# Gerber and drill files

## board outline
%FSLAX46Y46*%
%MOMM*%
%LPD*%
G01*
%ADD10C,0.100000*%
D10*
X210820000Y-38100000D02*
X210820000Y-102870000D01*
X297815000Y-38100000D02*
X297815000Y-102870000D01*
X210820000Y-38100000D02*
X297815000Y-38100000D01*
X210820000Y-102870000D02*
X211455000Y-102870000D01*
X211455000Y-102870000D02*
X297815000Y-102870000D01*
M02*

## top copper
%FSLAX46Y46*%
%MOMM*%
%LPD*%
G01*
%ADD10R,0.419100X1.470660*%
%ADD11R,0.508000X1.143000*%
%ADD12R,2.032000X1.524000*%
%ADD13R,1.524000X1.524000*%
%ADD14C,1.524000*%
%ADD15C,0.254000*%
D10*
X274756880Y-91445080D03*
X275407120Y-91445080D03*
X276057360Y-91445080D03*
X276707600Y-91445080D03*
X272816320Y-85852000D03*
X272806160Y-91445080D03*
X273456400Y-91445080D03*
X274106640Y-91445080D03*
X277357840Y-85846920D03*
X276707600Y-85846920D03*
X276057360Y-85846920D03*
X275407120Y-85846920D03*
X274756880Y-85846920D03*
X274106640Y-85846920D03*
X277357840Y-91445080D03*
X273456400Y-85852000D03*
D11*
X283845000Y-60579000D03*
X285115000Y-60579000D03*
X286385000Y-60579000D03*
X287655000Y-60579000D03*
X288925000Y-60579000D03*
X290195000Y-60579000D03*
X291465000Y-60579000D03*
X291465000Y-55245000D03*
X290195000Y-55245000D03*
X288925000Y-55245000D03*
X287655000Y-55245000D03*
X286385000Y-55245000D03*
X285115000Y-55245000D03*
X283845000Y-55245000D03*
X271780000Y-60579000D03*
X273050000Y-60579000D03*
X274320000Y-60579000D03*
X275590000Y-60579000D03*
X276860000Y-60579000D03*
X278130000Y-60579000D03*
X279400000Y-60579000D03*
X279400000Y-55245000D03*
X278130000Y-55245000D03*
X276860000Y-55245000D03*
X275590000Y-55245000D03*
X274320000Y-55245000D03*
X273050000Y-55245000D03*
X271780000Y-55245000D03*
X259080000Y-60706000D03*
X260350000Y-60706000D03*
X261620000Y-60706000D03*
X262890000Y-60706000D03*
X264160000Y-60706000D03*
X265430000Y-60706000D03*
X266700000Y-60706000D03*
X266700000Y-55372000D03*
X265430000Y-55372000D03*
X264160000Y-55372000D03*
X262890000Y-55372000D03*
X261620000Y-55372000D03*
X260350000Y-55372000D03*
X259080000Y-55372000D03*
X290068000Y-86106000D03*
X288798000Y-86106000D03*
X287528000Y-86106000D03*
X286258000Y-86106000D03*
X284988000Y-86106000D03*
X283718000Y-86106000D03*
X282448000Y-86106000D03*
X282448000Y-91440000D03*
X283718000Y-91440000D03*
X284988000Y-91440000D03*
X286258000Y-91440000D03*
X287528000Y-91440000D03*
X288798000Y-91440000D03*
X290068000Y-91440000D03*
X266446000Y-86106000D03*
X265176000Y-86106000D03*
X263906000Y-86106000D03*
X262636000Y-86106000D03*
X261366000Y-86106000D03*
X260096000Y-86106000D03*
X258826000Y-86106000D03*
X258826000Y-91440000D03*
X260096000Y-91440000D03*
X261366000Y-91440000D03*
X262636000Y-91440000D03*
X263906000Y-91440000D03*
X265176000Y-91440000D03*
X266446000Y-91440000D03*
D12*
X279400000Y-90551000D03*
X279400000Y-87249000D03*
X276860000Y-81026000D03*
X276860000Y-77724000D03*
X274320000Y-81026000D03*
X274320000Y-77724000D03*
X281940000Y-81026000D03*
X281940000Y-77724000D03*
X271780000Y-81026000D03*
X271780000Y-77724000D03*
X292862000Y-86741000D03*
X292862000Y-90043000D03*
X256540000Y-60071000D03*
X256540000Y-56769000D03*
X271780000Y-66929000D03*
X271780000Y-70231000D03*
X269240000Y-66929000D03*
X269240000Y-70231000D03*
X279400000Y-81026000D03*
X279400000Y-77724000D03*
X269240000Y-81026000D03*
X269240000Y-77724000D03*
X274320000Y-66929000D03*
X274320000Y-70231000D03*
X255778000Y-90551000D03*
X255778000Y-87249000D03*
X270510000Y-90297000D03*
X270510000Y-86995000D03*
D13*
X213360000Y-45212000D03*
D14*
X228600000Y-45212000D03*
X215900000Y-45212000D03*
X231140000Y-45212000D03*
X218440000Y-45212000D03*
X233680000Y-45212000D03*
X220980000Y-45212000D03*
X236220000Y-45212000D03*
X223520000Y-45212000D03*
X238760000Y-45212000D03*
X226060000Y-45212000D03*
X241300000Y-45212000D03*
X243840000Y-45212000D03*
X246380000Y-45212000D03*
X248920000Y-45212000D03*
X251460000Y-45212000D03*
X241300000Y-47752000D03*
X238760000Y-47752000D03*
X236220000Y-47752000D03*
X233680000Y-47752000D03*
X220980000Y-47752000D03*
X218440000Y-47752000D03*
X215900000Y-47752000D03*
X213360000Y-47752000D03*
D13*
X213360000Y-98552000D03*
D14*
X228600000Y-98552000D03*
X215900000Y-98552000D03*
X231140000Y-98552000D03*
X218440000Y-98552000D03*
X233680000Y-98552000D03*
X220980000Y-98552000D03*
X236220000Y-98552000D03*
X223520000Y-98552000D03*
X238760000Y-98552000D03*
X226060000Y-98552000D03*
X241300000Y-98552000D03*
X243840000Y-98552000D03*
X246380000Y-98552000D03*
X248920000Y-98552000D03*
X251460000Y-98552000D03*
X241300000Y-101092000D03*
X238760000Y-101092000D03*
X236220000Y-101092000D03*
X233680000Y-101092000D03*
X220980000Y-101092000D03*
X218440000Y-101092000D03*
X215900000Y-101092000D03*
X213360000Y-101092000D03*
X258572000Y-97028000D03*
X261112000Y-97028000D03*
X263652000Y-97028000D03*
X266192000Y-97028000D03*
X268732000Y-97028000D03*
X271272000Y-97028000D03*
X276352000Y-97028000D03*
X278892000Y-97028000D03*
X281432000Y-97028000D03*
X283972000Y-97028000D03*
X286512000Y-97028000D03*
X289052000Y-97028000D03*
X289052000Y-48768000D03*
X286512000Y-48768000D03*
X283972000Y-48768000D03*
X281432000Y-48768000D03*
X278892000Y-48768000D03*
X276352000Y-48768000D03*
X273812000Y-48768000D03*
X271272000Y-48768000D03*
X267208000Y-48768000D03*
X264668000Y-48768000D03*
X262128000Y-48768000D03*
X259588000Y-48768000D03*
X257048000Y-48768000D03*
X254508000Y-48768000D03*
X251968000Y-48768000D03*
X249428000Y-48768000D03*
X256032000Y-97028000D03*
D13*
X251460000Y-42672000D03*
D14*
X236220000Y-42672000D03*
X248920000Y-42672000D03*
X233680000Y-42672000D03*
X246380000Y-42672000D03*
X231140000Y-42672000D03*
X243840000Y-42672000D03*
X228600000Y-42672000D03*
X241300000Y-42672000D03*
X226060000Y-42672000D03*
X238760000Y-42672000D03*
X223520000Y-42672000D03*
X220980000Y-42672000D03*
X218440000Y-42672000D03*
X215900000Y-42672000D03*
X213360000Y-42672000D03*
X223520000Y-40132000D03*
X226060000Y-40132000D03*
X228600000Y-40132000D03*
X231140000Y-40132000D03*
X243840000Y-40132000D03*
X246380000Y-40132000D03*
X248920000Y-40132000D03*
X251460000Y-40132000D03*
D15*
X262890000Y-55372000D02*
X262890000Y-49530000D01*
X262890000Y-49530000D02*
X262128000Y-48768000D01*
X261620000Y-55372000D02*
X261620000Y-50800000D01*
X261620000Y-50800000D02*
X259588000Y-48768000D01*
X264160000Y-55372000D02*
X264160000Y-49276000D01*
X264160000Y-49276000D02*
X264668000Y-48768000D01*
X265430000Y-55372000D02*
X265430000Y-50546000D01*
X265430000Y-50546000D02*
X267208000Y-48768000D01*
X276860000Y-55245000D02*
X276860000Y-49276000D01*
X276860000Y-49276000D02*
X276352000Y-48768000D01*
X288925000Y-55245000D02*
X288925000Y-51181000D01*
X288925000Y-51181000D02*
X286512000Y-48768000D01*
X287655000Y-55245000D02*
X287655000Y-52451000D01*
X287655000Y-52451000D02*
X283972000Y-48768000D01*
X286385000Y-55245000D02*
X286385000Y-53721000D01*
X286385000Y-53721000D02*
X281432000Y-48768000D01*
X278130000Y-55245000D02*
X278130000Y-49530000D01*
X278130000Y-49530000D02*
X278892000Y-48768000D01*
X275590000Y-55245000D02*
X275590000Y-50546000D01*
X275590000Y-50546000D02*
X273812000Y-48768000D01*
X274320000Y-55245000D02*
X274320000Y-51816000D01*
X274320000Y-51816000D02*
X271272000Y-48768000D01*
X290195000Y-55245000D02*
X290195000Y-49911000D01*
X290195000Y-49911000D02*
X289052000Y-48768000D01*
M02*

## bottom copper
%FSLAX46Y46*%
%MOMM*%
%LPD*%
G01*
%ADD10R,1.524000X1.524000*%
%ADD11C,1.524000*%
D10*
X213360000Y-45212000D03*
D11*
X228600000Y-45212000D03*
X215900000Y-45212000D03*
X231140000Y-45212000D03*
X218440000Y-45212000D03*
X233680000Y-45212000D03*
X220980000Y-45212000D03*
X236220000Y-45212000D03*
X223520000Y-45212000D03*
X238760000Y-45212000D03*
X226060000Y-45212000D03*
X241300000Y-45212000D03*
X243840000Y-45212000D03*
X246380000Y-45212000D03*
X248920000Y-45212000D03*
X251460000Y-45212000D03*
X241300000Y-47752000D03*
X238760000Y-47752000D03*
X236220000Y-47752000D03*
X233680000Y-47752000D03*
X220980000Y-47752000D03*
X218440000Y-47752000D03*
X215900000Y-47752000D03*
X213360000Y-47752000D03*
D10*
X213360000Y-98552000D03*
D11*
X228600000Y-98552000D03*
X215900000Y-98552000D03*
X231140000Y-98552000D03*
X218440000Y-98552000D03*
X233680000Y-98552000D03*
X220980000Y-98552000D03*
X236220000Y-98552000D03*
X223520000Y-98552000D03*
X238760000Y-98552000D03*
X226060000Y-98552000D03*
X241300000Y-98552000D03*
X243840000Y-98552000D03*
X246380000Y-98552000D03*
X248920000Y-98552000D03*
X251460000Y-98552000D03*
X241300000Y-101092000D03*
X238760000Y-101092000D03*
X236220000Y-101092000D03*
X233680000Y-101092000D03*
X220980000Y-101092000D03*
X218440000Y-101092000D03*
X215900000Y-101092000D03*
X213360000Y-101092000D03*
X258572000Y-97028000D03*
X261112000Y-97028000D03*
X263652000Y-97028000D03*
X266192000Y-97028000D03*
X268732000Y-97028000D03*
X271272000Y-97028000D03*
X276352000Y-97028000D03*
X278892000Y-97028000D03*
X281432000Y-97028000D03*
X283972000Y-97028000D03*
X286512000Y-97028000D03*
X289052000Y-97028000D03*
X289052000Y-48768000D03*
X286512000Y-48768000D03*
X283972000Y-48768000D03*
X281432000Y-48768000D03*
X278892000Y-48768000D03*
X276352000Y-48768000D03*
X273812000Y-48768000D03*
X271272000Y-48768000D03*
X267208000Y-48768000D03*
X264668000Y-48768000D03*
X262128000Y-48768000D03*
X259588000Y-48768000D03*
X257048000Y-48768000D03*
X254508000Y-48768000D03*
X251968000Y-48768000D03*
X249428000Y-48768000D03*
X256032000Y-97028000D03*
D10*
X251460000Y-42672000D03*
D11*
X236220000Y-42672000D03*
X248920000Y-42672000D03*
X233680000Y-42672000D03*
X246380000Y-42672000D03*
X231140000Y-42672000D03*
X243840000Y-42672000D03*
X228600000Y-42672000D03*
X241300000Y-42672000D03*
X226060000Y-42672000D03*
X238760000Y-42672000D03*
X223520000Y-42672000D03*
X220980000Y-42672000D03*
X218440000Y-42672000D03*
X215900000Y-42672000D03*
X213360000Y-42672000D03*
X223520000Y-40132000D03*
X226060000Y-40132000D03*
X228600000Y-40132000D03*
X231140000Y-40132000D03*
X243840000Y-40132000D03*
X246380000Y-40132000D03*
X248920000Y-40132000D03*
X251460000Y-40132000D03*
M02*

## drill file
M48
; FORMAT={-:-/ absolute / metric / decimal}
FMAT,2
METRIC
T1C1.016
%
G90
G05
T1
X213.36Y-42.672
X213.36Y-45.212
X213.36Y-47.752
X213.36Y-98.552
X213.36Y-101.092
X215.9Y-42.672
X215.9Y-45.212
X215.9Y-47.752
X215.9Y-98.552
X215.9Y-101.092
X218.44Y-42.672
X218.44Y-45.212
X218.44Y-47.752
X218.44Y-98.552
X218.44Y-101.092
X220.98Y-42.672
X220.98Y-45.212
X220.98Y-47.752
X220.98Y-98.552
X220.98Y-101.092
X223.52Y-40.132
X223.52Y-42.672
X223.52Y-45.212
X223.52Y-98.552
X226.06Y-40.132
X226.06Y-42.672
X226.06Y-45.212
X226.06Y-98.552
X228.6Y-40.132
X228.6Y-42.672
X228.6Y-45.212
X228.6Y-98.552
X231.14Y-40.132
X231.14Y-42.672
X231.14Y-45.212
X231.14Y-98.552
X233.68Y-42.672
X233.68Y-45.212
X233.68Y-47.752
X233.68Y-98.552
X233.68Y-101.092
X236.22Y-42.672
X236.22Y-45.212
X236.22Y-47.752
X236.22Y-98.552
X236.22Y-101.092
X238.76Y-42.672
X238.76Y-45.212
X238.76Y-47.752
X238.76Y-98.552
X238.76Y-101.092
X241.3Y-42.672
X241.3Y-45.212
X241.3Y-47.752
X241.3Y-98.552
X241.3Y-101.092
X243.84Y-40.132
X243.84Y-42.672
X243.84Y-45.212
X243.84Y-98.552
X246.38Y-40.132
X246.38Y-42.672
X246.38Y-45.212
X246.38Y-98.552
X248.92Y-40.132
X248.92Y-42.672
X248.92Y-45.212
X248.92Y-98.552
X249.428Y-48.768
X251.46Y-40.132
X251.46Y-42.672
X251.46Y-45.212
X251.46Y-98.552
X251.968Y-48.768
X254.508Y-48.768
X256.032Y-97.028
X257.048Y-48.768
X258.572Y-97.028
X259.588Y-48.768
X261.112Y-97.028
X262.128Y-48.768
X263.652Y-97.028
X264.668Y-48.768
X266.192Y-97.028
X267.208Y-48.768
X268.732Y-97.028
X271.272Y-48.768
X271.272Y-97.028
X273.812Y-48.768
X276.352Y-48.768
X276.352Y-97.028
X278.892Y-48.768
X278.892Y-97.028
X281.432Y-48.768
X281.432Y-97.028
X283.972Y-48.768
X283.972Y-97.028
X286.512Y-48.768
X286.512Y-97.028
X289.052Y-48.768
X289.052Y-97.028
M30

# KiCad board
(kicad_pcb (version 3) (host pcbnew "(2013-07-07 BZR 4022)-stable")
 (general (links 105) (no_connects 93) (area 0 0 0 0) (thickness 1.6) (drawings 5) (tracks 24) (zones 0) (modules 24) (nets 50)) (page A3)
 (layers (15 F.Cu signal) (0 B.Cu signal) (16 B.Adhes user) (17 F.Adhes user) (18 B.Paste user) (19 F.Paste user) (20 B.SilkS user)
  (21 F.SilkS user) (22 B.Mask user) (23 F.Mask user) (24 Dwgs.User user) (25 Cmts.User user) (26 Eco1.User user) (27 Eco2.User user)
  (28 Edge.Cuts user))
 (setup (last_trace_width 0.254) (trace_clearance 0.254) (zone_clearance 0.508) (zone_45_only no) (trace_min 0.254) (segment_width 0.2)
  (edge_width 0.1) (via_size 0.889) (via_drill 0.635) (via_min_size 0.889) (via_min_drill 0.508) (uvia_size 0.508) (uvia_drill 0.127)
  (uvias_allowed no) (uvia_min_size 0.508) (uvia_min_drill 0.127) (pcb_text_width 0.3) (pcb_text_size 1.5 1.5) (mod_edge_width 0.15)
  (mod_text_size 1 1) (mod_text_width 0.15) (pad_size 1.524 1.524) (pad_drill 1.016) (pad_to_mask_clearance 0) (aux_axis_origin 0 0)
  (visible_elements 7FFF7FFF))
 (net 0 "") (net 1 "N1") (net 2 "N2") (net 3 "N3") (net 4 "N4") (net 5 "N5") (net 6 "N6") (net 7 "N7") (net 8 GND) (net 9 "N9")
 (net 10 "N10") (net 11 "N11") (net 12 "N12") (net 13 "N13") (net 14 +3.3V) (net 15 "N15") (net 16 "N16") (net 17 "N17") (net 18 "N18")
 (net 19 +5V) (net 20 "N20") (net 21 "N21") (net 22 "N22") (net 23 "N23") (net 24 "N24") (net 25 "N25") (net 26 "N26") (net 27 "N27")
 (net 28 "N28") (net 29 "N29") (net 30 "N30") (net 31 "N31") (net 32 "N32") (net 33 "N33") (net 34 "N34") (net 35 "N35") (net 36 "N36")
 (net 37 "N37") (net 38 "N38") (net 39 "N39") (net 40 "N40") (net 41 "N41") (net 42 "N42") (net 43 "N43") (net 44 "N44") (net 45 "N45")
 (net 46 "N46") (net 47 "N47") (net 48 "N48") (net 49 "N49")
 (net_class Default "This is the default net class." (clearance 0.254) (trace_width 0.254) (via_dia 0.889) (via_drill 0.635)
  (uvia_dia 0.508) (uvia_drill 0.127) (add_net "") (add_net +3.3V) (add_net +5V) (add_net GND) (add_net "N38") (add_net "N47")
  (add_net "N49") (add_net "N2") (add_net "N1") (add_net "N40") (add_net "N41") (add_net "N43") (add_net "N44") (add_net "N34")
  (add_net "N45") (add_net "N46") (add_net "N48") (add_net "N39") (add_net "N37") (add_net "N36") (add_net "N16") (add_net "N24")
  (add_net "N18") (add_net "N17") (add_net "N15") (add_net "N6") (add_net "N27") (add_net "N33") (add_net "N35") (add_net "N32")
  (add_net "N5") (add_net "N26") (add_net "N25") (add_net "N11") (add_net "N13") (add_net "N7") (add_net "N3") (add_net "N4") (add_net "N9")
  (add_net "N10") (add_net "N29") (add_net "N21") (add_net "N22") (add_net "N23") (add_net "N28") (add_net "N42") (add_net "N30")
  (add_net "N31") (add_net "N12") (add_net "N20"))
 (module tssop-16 (layer F.Cu) (at 275.082 88.646)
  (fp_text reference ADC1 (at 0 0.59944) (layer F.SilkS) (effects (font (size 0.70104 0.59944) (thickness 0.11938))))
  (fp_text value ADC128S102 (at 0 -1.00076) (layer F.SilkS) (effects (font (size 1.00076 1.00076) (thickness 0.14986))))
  (pad 4 smd rect (at -0.32512 2.79908) (size 0.4191 1.47066) (layers F.Cu F.Paste F.Mask) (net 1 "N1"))
  (pad 5 smd rect (at 0.32512 2.79908) (size 0.4191 1.47066) (layers F.Cu F.Paste F.Mask) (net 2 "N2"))
  (pad 6 smd rect (at 0.97536 2.79908) (size 0.4191 1.47066) (layers F.Cu F.Paste F.Mask) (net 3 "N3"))
  (pad 7 smd rect (at 1.6256 2.79908) (size 0.4191 1.47066) (layers F.Cu F.Paste F.Mask) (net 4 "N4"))
  (pad 16 smd rect (at -2.26568 -2.794) (size 0.4191 1.47066) (layers F.Cu F.Paste F.Mask) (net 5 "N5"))
  (pad 1 smd rect (at -2.27584 2.79908) (size 0.4191 1.47066) (layers F.Cu F.Paste F.Mask) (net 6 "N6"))
  (pad 2 smd rect (at -1.6256 2.79908) (size 0.4191 1.47066) (layers F.Cu F.Paste F.Mask) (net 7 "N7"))
  (pad 3 smd rect (at -0.97536 2.79908) (size 0.4191 1.47066) (layers F.Cu F.Paste F.Mask) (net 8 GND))
  (pad 9 smd rect (at 2.27584 -2.79908) (size 0.4191 1.47066) (layers F.Cu F.Paste F.Mask) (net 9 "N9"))
  (pad 10 smd rect (at 1.6256 -2.79908) (size 0.4191 1.47066) (layers F.Cu F.Paste F.Mask))
  (pad 11 smd rect (at 0.97536 -2.79908) (size 0.4191 1.47066) (layers F.Cu F.Paste F.Mask))
  (pad 12 smd rect (at 0.32512 -2.79908) (size 0.4191 1.47066) (layers F.Cu F.Paste F.Mask) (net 8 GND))
  (pad 13 smd rect (at -0.32512 -2.79908) (size 0.4191 1.47066) (layers F.Cu F.Paste F.Mask) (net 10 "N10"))
  (pad 14 smd rect (at -0.97536 -2.79908) (size 0.4191 1.47066) (layers F.Cu F.Paste F.Mask) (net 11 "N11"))
  (pad 8 smd rect (at 2.27584 2.79908) (size 0.4191 1.47066) (layers F.Cu F.Paste F.Mask) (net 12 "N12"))
  (pad 15 smd rect (at -1.6256 -2.794) (size 0.4191 1.47066) (layers F.Cu F.Paste F.Mask) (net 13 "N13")))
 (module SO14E (layer F.Cu) (at 287.655 57.785)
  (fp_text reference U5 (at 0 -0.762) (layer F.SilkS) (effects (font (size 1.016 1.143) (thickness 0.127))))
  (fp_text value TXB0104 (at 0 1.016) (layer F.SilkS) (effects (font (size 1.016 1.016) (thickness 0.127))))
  (pad 1 smd rect (at -3.81 2.794) (size 0.508 1.143) (layers F.Cu F.Paste F.Mask) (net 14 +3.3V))
  (pad 2 smd rect (at -2.54 2.794) (size 0.508 1.143) (layers F.Cu F.Paste F.Mask) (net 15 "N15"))
  (pad 3 smd rect (at -1.27 2.794) (size 0.508 1.143) (layers F.Cu F.Paste F.Mask) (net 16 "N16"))
  (pad 4 smd rect (at 0 2.794) (size 0.508 1.143) (layers F.Cu F.Paste F.Mask) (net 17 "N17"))
  (pad 5 smd rect (at 1.27 2.794) (size 0.508 1.143) (layers F.Cu F.Paste F.Mask) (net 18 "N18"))
  (pad 6 smd rect (at 2.54 2.794) (size 0.508 1.143) (layers F.Cu F.Paste F.Mask))
  (pad 7 smd rect (at 3.81 2.794) (size 0.508 1.143) (layers F.Cu F.Paste F.Mask) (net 8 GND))
  (pad 8 smd rect (at 3.81 -2.54) (size 0.508 1.143) (layers F.Cu F.Paste F.Mask) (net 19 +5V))
  (pad 9 smd rect (at 2.54 -2.54) (size 0.508 1.143) (layers F.Cu F.Paste F.Mask) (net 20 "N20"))
  (pad 10 smd rect (at 1.27 -2.54) (size 0.508 1.143) (layers F.Cu F.Paste F.Mask) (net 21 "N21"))
  (pad 11 smd rect (at 0 -2.54) (size 0.508 1.143) (layers F.Cu F.Paste F.Mask) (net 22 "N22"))
  (pad 12 smd rect (at -1.27 -2.54) (size 0.508 1.143) (layers F.Cu F.Paste F.Mask) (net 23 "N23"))
  (pad 13 smd rect (at -2.54 -2.54) (size 0.508 1.143) (layers F.Cu F.Paste F.Mask))
  (pad 14 smd rect (at -3.81 -2.54) (size 0.508 1.143) (layers F.Cu F.Paste F.Mask)))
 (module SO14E (layer F.Cu) (at 275.59 57.785)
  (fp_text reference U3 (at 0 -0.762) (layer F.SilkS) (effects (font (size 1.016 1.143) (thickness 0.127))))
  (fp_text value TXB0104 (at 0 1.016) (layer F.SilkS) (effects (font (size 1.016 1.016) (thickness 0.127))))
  (pad 1 smd rect (at -3.81 2.794) (size 0.508 1.143) (layers F.Cu F.Paste F.Mask) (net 14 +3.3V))
  (pad 2 smd rect (at -2.54 2.794) (size 0.508 1.143) (layers F.Cu F.Paste F.Mask) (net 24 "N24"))
  (pad 3 smd rect (at -1.27 2.794) (size 0.508 1.143) (layers F.Cu F.Paste F.Mask) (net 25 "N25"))
  (pad 4 smd rect (at 0 2.794) (size 0.508 1.143) (layers F.Cu F.Paste F.Mask) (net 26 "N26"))
  (pad 5 smd rect (at 1.27 2.794) (size 0.508 1.143) (layers F.Cu F.Paste F.Mask) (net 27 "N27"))
  (pad 6 smd rect (at 2.54 2.794) (size 0.508 1.143) (layers F.Cu F.Paste F.Mask))
  (pad 7 smd rect (at 3.81 2.794) (size 0.508 1.143) (layers F.Cu F.Paste F.Mask) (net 8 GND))
  (pad 8 smd rect (at 3.81 -2.54) (size 0.508 1.143) (layers F.Cu F.Paste F.Mask) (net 19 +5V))
  (pad 9 smd rect (at 2.54 -2.54) (size 0.508 1.143) (layers F.Cu F.Paste F.Mask) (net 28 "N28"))
  (pad 10 smd rect (at 1.27 -2.54) (size 0.508 1.143) (layers F.Cu F.Paste F.Mask) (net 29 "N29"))
  (pad 11 smd rect (at 0 -2.54) (size 0.508 1.143) (layers F.Cu F.Paste F.Mask) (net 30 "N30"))
  (pad 12 smd rect (at -1.27 -2.54) (size 0.508 1.143) (layers F.Cu F.Paste F.Mask) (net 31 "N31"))
  (pad 13 smd rect (at -2.54 -2.54) (size 0.508 1.143) (layers F.Cu F.Paste F.Mask))
  (pad 14 smd rect (at -3.81 -2.54) (size 0.508 1.143) (layers F.Cu F.Paste F.Mask)))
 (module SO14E (layer F.Cu) (at 262.89 57.912)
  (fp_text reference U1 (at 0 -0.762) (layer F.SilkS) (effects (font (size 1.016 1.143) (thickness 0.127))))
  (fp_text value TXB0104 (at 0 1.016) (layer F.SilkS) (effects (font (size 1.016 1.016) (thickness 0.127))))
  (pad 1 smd rect (at -3.81 2.794) (size 0.508 1.143) (layers F.Cu F.Paste F.Mask) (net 14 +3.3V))
  (pad 2 smd rect (at -2.54 2.794) (size 0.508 1.143) (layers F.Cu F.Paste F.Mask) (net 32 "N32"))
  (pad 3 smd rect (at -1.27 2.794) (size 0.508 1.143) (layers F.Cu F.Paste F.Mask) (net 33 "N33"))
  (pad 4 smd rect (at 0 2.794) (size 0.508 1.143) (layers F.Cu F.Paste F.Mask) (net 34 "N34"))
  (pad 5 smd rect (at 1.27 2.794) (size 0.508 1.143) (layers F.Cu F.Paste F.Mask) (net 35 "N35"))
  (pad 6 smd rect (at 2.54 2.794) (size 0.508 1.143) (layers F.Cu F.Paste F.Mask))
  (pad 7 smd rect (at 3.81 2.794) (size 0.508 1.143) (layers F.Cu F.Paste F.Mask))
  (pad 8 smd rect (at 3.81 -2.54) (size 0.508 1.143) (layers F.Cu F.Paste F.Mask) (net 19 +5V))
  (pad 9 smd rect (at 2.54 -2.54) (size 0.508 1.143) (layers F.Cu F.Paste F.Mask) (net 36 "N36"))
  (pad 10 smd rect (at 1.27 -2.54) (size 0.508 1.143) (layers F.Cu F.Paste F.Mask) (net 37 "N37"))
  (pad 11 smd rect (at 0 -2.54) (size 0.508 1.143) (layers F.Cu F.Paste F.Mask) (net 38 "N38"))
  (pad 12 smd rect (at -1.27 -2.54) (size 0.508 1.143) (layers F.Cu F.Paste F.Mask) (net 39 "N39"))
  (pad 13 smd rect (at -2.54 -2.54) (size 0.508 1.143) (layers F.Cu F.Paste F.Mask))
  (pad 14 smd rect (at -3.81 -2.54) (size 0.508 1.143) (layers F.Cu F.Paste F.Mask)))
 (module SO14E (layer F.Cu) (at 286.258 88.9 180)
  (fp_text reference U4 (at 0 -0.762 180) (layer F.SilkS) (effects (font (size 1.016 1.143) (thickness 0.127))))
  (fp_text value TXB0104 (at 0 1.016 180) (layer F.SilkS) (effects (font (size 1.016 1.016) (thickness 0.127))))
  (pad 1 smd rect (at -3.81 2.794 180) (size 0.508 1.143) (layers F.Cu F.Paste F.Mask) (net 14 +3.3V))
  (pad 2 smd rect (at -2.54 2.794 180) (size 0.508 1.143) (layers F.Cu F.Paste F.Mask) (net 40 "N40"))
  (pad 3 smd rect (at -1.27 2.794 180) (size 0.508 1.143) (layers F.Cu F.Paste F.Mask) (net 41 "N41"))
  (pad 4 smd rect (at 0 2.794 180) (size 0.508 1.143) (layers F.Cu F.Paste F.Mask) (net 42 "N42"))
  (pad 5 smd rect (at 1.27 2.794 180) (size 0.508 1.143) (layers F.Cu F.Paste F.Mask) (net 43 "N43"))
  (pad 6 smd rect (at 2.54 2.794 180) (size 0.508 1.143) (layers F.Cu F.Paste F.Mask))
  (pad 7 smd rect (at 3.81 2.794 180) (size 0.508 1.143) (layers F.Cu F.Paste F.Mask) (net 8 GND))
  (pad 8 smd rect (at 3.81 -2.54 180) (size 0.508 1.143) (layers F.Cu F.Paste F.Mask) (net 19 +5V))
  (pad 9 smd rect (at 2.54 -2.54 180) (size 0.508 1.143) (layers F.Cu F.Paste F.Mask) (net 3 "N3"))
  (pad 10 smd rect (at 1.27 -2.54 180) (size 0.508 1.143) (layers F.Cu F.Paste F.Mask) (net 4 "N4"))
  (pad 11 smd rect (at 0 -2.54 180) (size 0.508 1.143) (layers F.Cu F.Paste F.Mask) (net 12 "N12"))
  (pad 12 smd rect (at -1.27 -2.54 180) (size 0.508 1.143) (layers F.Cu F.Paste F.Mask) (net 9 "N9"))
  (pad 13 smd rect (at -2.54 -2.54 180) (size 0.508 1.143) (layers F.Cu F.Paste F.Mask))
  (pad 14 smd rect (at -3.81 -2.54 180) (size 0.508 1.143) (layers F.Cu F.Paste F.Mask)))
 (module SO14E (layer F.Cu) (at 262.636 88.9 180)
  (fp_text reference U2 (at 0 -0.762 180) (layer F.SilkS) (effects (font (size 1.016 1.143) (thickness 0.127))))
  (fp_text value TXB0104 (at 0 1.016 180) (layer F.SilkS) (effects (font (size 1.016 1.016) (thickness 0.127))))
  (pad 1 smd rect (at -3.81 2.794 180) (size 0.508 1.143) (layers F.Cu F.Paste F.Mask) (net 14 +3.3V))
  (pad 2 smd rect (at -2.54 2.794 180) (size 0.508 1.143) (layers F.Cu F.Paste F.Mask) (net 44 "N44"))
  (pad 3 smd rect (at -1.27 2.794 180) (size 0.508 1.143) (layers F.Cu F.Paste F.Mask) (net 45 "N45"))
  (pad 4 smd rect (at 0 2.794 180) (size 0.508 1.143) (layers F.Cu F.Paste F.Mask) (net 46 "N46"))
  (pad 5 smd rect (at 1.27 2.794 180) (size 0.508 1.143) (layers F.Cu F.Paste F.Mask) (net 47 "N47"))
  (pad 6 smd rect (at 2.54 2.794 180) (size 0.508 1.143) (layers F.Cu F.Paste F.Mask))
  (pad 7 smd rect (at 3.81 2.794 180) (size 0.508 1.143) (layers F.Cu F.Paste F.Mask) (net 8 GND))
  (pad 8 smd rect (at 3.81 -2.54 180) (size 0.508 1.143) (layers F.Cu F.Paste F.Mask) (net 19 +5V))
  (pad 9 smd rect (at 2.54 -2.54 180) (size 0.508 1.143) (layers F.Cu F.Paste F.Mask) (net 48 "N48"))
  (pad 10 smd rect (at 1.27 -2.54 180) (size 0.508 1.143) (layers F.Cu F.Paste F.Mask) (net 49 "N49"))
  (pad 11 smd rect (at 0 -2.54 180) (size 0.508 1.143) (layers F.Cu F.Paste F.Mask) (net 1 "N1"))
  (pad 12 smd rect (at -1.27 -2.54 180) (size 0.508 1.143) (layers F.Cu F.Paste F.Mask) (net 2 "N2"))
  (pad 13 smd rect (at -2.54 -2.54 180) (size 0.508 1.143) (layers F.Cu F.Paste F.Mask))
  (pad 14 smd rect (at -3.81 -2.54 180) (size 0.508 1.143) (layers F.Cu F.Paste F.Mask)))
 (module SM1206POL (layer F.Cu) (at 279.4 88.9 90)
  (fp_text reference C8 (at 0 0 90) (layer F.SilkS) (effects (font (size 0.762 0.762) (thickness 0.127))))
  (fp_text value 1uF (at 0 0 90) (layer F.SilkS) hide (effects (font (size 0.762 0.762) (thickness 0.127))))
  (pad 1 smd rect (at -1.651 0 90) (size 1.524 2.032) (layers F.Cu F.Paste F.Mask) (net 7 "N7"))
  (pad 2 smd rect (at 1.651 0 90) (size 1.524 2.032) (layers F.Cu F.Paste F.Mask) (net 8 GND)))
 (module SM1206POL (layer F.Cu) (at 276.86 79.375 90)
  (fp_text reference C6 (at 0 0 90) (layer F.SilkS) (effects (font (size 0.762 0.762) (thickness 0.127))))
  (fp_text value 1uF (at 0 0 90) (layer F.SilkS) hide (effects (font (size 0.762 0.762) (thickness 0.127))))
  (pad 1 smd rect (at -1.651 0 90) (size 1.524 2.032) (layers F.Cu F.Paste F.Mask) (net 10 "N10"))
  (pad 2 smd rect (at 1.651 0 90) (size 1.524 2.032) (layers F.Cu F.Paste F.Mask) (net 8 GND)))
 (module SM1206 (layer F.Cu) (at 274.32 79.375 90)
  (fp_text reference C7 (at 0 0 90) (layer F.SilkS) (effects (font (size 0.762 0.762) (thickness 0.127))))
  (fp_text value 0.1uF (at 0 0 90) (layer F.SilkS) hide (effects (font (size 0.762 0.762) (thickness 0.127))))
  (pad 1 smd rect (at -1.651 0 90) (size 1.524 2.032) (layers F.Cu F.Paste F.Mask) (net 10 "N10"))
  (pad 2 smd rect (at 1.651 0 90) (size 1.524 2.032) (layers F.Cu F.Paste F.Mask) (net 8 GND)))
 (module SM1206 (layer F.Cu) (at 281.94 79.375 90)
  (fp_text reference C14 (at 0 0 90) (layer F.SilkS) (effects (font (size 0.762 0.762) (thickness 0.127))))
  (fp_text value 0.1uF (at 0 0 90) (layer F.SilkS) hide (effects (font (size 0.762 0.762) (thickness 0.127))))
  (pad 1 smd rect (at -1.651 0 90) (size 1.524 2.032) (layers F.Cu F.Paste F.Mask) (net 14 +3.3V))
  (pad 2 smd rect (at 1.651 0 90) (size 1.524 2.032) (layers F.Cu F.Paste F.Mask) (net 8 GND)))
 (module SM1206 (layer F.Cu) (at 271.78 79.375 90)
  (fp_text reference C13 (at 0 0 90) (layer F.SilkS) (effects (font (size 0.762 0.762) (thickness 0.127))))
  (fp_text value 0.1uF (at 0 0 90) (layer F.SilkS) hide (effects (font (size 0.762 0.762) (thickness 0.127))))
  (pad 1 smd rect (at -1.651 0 90) (size 1.524 2.032) (layers F.Cu F.Paste F.Mask) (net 14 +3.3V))
  (pad 2 smd rect (at 1.651 0 90) (size 1.524 2.032) (layers F.Cu F.Paste F.Mask) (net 8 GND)))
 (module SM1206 (layer F.Cu) (at 292.862 88.392 270)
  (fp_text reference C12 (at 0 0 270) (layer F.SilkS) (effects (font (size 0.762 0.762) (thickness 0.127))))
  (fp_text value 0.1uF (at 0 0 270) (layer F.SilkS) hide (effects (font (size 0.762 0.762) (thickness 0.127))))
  (pad 1 smd rect (at -1.651 0 270) (size 1.524 2.032) (layers F.Cu F.Paste F.Mask) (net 14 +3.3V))
  (pad 2 smd rect (at 1.651 0 270) (size 1.524 2.032) (layers F.Cu F.Paste F.Mask) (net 8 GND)))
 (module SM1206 (layer F.Cu) (at 256.54 58.42 90)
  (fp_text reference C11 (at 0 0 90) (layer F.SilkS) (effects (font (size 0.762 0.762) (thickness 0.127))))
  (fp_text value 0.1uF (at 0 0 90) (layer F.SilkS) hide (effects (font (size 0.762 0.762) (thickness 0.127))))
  (pad 1 smd rect (at -1.651 0 90) (size 1.524 2.032) (layers F.Cu F.Paste F.Mask) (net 14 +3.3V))
  (pad 2 smd rect (at 1.651 0 90) (size 1.524 2.032) (layers F.Cu F.Paste F.Mask) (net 8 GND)))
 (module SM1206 (layer F.Cu) (at 271.78 68.58 270)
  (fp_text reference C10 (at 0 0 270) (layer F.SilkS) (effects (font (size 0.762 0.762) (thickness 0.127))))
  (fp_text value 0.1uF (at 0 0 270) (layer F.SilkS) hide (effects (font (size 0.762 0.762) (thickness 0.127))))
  (pad 1 smd rect (at -1.651 0 270) (size 1.524 2.032) (layers F.Cu F.Paste F.Mask) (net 14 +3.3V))
  (pad 2 smd rect (at 1.651 0 270) (size 1.524 2.032) (layers F.Cu F.Paste F.Mask) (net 8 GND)))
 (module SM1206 (layer F.Cu) (at 269.24 68.58 270)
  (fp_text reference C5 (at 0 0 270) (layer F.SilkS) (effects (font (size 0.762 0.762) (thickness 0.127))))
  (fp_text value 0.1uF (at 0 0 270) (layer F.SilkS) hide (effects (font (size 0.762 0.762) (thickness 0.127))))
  (pad 1 smd rect (at -1.651 0 270) (size 1.524 2.032) (layers F.Cu F.Paste F.Mask) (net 19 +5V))
  (pad 2 smd rect (at 1.651 0 270) (size 1.524 2.032) (layers F.Cu F.Paste F.Mask) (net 8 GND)))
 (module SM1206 (layer F.Cu) (at 279.4 79.375 90)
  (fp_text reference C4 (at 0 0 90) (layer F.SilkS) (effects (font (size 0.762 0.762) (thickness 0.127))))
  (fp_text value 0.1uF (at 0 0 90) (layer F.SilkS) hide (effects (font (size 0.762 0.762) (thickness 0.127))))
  (pad 1 smd rect (at -1.651 0 90) (size 1.524 2.032) (layers F.Cu F.Paste F.Mask) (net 19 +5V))
  (pad 2 smd rect (at 1.651 0 90) (size 1.524 2.032) (layers F.Cu F.Paste F.Mask) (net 8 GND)))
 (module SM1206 (layer F.Cu) (at 269.24 79.375 90)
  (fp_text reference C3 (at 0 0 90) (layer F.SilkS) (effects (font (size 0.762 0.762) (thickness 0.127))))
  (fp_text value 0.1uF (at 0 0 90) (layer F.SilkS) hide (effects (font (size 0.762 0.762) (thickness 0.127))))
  (pad 1 smd rect (at -1.651 0 90) (size 1.524 2.032) (layers F.Cu F.Paste F.Mask) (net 19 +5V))
  (pad 2 smd rect (at 1.651 0 90) (size 1.524 2.032) (layers F.Cu F.Paste F.Mask) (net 8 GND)))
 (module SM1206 (layer F.Cu) (at 274.32 68.58 270)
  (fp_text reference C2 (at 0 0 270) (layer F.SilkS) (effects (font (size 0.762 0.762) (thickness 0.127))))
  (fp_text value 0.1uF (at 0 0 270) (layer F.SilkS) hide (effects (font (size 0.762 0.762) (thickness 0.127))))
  (pad 1 smd rect (at -1.651 0 270) (size 1.524 2.032) (layers F.Cu F.Paste F.Mask) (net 19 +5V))
  (pad 2 smd rect (at 1.651 0 270) (size 1.524 2.032) (layers F.Cu F.Paste F.Mask) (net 8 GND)))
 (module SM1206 (layer F.Cu) (at 255.778 88.9 90)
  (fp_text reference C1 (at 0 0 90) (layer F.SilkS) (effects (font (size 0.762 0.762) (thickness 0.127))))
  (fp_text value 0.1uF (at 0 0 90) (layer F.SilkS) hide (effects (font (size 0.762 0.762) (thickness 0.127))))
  (pad 1 smd rect (at -1.651 0 90) (size 1.524 2.032) (layers F.Cu F.Paste F.Mask) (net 19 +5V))
  (pad 2 smd rect (at 1.651 0 90) (size 1.524 2.032) (layers F.Cu F.Paste F.Mask) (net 8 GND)))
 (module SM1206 (layer F.Cu) (at 270.51 88.646 90)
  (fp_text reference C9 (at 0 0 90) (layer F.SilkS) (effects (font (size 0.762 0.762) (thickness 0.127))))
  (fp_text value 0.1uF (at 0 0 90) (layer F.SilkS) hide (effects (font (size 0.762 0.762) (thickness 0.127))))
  (pad 1 smd rect (at -1.651 0 90) (size 1.524 2.032) (layers F.Cu F.Paste F.Mask) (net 7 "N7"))
  (pad 2 smd rect (at 1.651 0 90) (size 1.524 2.032) (layers F.Cu F.Paste F.Mask) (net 8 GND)))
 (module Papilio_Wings (layer F.Cu) (at 234.95 46.482)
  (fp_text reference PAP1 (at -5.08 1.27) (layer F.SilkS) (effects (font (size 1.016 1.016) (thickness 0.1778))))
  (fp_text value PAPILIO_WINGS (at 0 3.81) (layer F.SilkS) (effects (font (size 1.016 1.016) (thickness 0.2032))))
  (pad 1 thru_hole rect (at -21.59 -1.27) (size 1.524 1.524) (drill 1.016) (layers *.Cu *.Mask F.SilkS) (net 35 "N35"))
  (pad 7 thru_hole circle (at -6.35 -1.27) (size 1.524 1.524) (drill 1.016) (layers *.Cu *.Mask F.SilkS) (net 25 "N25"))
  (pad 2 thru_hole circle (at -19.05 -1.27) (size 1.524 1.524) (drill 1.016) (layers *.Cu *.Mask F.SilkS) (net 34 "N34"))
  (pad 8 thru_hole circle (at -3.81 -1.27) (size 1.524 1.524) (drill 1.016) (layers *.Cu *.Mask F.SilkS) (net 24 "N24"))
  (pad 3 thru_hole circle (at -16.51 -1.27) (size 1.524 1.524) (drill 1.016) (layers *.Cu *.Mask F.SilkS) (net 33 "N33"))
  (pad 9 thru_hole circle (at -1.27 -1.27) (size 1.524 1.524) (drill 1.016) (layers *.Cu *.Mask F.SilkS) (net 18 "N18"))
  (pad 4 thru_hole circle (at -13.97 -1.27) (size 1.524 1.524) (drill 1.016) (layers *.Cu *.Mask F.SilkS) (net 32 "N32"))
  (pad 10 thru_hole circle (at 1.27 -1.27) (size 1.524 1.524) (drill 1.016) (layers *.Cu *.Mask F.SilkS) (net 17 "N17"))
  (pad 5 thru_hole circle (at -11.43 -1.27) (size 1.524 1.524) (drill 1.016) (layers *.Cu *.Mask F.SilkS) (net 27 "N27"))
  (pad 11 thru_hole circle (at 3.81 -1.27) (size 1.524 1.524) (drill 1.016) (layers *.Cu *.Mask F.SilkS) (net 16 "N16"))
  (pad 6 thru_hole circle (at -8.89 -1.27) (size 1.524 1.524) (drill 1.016) (layers *.Cu *.Mask F.SilkS) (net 26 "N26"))
  (pad 12 thru_hole circle (at 6.35 -1.27) (size 1.524 1.524) (drill 1.016) (layers *.Cu *.Mask F.SilkS) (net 15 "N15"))
  (pad 13 thru_hole circle (at 8.89 -1.27) (size 1.524 1.524) (drill 1.016) (layers *.Cu *.Mask F.SilkS))
  (pad 14 thru_hole circle (at 11.43 -1.27) (size 1.524 1.524) (drill 1.016) (layers *.Cu *.Mask F.SilkS))
  (pad 15 thru_hole circle (at 13.97 -1.27) (size 1.524 1.524) (drill 1.016) (layers *.Cu *.Mask F.SilkS))
  (pad 16 thru_hole circle (at 16.51 -1.27) (size 1.524 1.524) (drill 1.016) (layers *.Cu *.Mask F.SilkS))
  (pad 17 thru_hole circle (at 6.35 1.27) (size 1.524 1.524) (drill 1.016) (layers *.Cu *.Mask F.SilkS) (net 19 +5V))
  (pad 18 thru_hole circle (at 3.81 1.27) (size 1.524 1.524) (drill 1.016) (layers *.Cu *.Mask F.SilkS) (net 14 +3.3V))
  (pad 19 thru_hole circle (at 1.27 1.27) (size 1.524 1.524) (drill 1.016) (layers *.Cu *.Mask F.SilkS))
  (pad 20 thru_hole circle (at -1.27 1.27) (size 1.524 1.524) (drill 1.016) (layers *.Cu *.Mask F.SilkS) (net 8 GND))
  (pad 21 thru_hole circle (at -13.97 1.27) (size 1.524 1.524) (drill 1.016) (layers *.Cu *.Mask F.SilkS) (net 19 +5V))
  (pad 22 thru_hole circle (at -16.51 1.27) (size 1.524 1.524) (drill 1.016) (layers *.Cu *.Mask F.SilkS))
  (pad 23 thru_hole circle (at -19.05 1.27) (size 1.524 1.524) (drill 1.016) (layers *.Cu *.Mask F.SilkS) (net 14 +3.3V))
  (pad 24 thru_hole circle (at -21.59 1.27) (size 1.524 1.524) (drill 1.016) (layers *.Cu *.Mask F.SilkS) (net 8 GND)))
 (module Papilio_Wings (layer F.Cu) (at 234.95 99.822)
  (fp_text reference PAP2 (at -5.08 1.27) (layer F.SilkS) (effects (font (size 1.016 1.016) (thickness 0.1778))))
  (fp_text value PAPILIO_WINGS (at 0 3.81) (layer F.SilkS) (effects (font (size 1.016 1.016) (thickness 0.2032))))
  (pad 1 thru_hole rect (at -21.59 -1.27) (size 1.524 1.524) (drill 1.016) (layers *.Cu *.Mask F.SilkS))
  (pad 7 thru_hole circle (at -6.35 -1.27) (size 1.524 1.524) (drill 1.016) (layers *.Cu *.Mask F.SilkS) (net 5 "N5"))
  (pad 2 thru_hole circle (at -19.05 -1.27) (size 1.524 1.524) (drill 1.016) (layers *.Cu *.Mask F.SilkS))
  (pad 8 thru_hole circle (at -3.81 -1.27) (size 1.524 1.524) (drill 1.016) (layers *.Cu *.Mask F.SilkS) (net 6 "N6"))
  (pad 3 thru_hole circle (at -16.51 -1.27) (size 1.524 1.524) (drill 1.016) (layers *.Cu *.Mask F.SilkS))
  (pad 9 thru_hole circle (at -1.27 -1.27) (size 1.524 1.524) (drill 1.016) (layers *.Cu *.Mask F.SilkS) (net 43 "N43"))
  (pad 4 thru_hole circle (at -13.97 -1.27) (size 1.524 1.524) (drill 1.016) (layers *.Cu *.Mask F.SilkS))
  (pad 10 thru_hole circle (at 1.27 -1.27) (size 1.524 1.524) (drill 1.016) (layers *.Cu *.Mask F.SilkS) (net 42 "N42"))
  (pad 5 thru_hole circle (at -11.43 -1.27) (size 1.524 1.524) (drill 1.016) (layers *.Cu *.Mask F.SilkS) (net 13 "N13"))
  (pad 11 thru_hole circle (at 3.81 -1.27) (size 1.524 1.524) (drill 1.016) (layers *.Cu *.Mask F.SilkS) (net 41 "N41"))
  (pad 6 thru_hole circle (at -8.89 -1.27) (size 1.524 1.524) (drill 1.016) (layers *.Cu *.Mask F.SilkS) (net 11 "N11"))
  (pad 12 thru_hole circle (at 6.35 -1.27) (size 1.524 1.524) (drill 1.016) (layers *.Cu *.Mask F.SilkS) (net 40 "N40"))
  (pad 13 thru_hole circle (at 8.89 -1.27) (size 1.524 1.524) (drill 1.016) (layers *.Cu *.Mask F.SilkS) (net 47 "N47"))
  (pad 14 thru_hole circle (at 11.43 -1.27) (size 1.524 1.524) (drill 1.016) (layers *.Cu *.Mask F.SilkS) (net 46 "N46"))
  (pad 15 thru_hole circle (at 13.97 -1.27) (size 1.524 1.524) (drill 1.016) (layers *.Cu *.Mask F.SilkS) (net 45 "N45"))
  (pad 16 thru_hole circle (at 16.51 -1.27) (size 1.524 1.524) (drill 1.016) (layers *.Cu *.Mask F.SilkS) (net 44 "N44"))
  (pad 17 thru_hole circle (at 6.35 1.27) (size 1.524 1.524) (drill 1.016) (layers *.Cu *.Mask F.SilkS) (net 19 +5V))
  (pad 18 thru_hole circle (at 3.81 1.27) (size 1.524 1.524) (drill 1.016) (layers *.Cu *.Mask F.SilkS) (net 14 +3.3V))
  (pad 19 thru_hole circle (at 1.27 1.27) (size 1.524 1.524) (drill 1.016) (layers *.Cu *.Mask F.SilkS))
  (pad 20 thru_hole circle (at -1.27 1.27) (size 1.524 1.524) (drill 1.016) (layers *.Cu *.Mask F.SilkS) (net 8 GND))
  (pad 21 thru_hole circle (at -13.97 1.27) (size 1.524 1.524) (drill 1.016) (layers *.Cu *.Mask F.SilkS) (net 19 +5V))
  (pad 22 thru_hole circle (at -16.51 1.27) (size 1.524 1.524) (drill 1.016) (layers *.Cu *.Mask F.SilkS) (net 14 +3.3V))
  (pad 23 thru_hole circle (at -19.05 1.27) (size 1.524 1.524) (drill 1.016) (layers *.Cu *.Mask F.SilkS))
  (pad 24 thru_hole circle (at -21.59 1.27) (size 1.524 1.524) (drill 1.016) (layers *.Cu *.Mask F.SilkS) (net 8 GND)))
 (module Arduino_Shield (layer F.Cu) (at 271.272 72.644)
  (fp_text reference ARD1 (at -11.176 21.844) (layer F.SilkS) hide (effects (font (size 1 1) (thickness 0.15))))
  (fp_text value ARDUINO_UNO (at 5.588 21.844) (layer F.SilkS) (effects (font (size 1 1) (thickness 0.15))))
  (pad 2 thru_hole circle (at -12.7 24.384) (size 1.524 1.524) (drill 1.016) (layers *.Cu *.Mask F.SilkS))
  (pad 3 thru_hole circle (at -10.16 24.384) (size 1.524 1.524) (drill 1.016) (layers *.Cu *.Mask F.SilkS) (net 14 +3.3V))
  (pad 4 thru_hole circle (at -7.62 24.384) (size 1.524 1.524) (drill 1.016) (layers *.Cu *.Mask F.SilkS) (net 19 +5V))
  (pad 5 thru_hole circle (at -5.08 24.384) (size 1.524 1.524) (drill 1.016) (layers *.Cu *.Mask F.SilkS))
  (pad 6 thru_hole circle (at -2.54 24.384) (size 1.524 1.524) (drill 1.016) (layers *.Cu *.Mask F.SilkS))
  (pad 7 thru_hole circle (at 0 24.384) (size 1.524 1.524) (drill 1.016) (layers *.Cu *.Mask F.SilkS))
  (pad 8 thru_hole circle (at 5.08 24.384) (size 1.524 1.524) (drill 1.016) (layers *.Cu *.Mask F.SilkS) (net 1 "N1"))
  (pad 9 thru_hole circle (at 7.62 24.384) (size 1.524 1.524) (drill 1.016) (layers *.Cu *.Mask F.SilkS) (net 2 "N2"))
  (pad 10 thru_hole circle (at 10.16 24.384) (size 1.524 1.524) (drill 1.016) (layers *.Cu *.Mask F.SilkS) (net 3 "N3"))
  (pad 11 thru_hole circle (at 12.7 24.384) (size 1.524 1.524) (drill 1.016) (layers *.Cu *.Mask F.SilkS) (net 4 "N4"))
  (pad 12 thru_hole circle (at 15.24 24.384) (size 1.524 1.524) (drill 1.016) (layers *.Cu *.Mask F.SilkS) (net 12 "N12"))
  (pad 13 thru_hole circle (at 17.78 24.384) (size 1.524 1.524) (drill 1.016) (layers *.Cu *.Mask F.SilkS) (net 9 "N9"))
  (pad 14 thru_hole circle (at 17.78 -23.876) (size 1.524 1.524) (drill 1.016) (layers *.Cu *.Mask F.SilkS) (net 20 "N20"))
  (pad 15 thru_hole circle (at 15.24 -23.876) (size 1.524 1.524) (drill 1.016) (layers *.Cu *.Mask F.SilkS) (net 21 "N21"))
  (pad 16 thru_hole circle (at 12.7 -23.876) (size 1.524 1.524) (drill 1.016) (layers *.Cu *.Mask F.SilkS) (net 22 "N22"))
  (pad 17 thru_hole circle (at 10.16 -23.876) (size 1.524 1.524) (drill 1.016) (layers *.Cu *.Mask F.SilkS) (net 23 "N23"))
  (pad 18 thru_hole circle (at 7.62 -23.876) (size 1.524 1.524) (drill 1.016) (layers *.Cu *.Mask F.SilkS) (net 28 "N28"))
  (pad 19 thru_hole circle (at 5.08 -23.876) (size 1.524 1.524) (drill 1.016) (layers *.Cu *.Mask F.SilkS) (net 29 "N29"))
  (pad 20 thru_hole circle (at 2.54 -23.876) (size 1.524 1.524) (drill 1.016) (layers *.Cu *.Mask F.SilkS) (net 30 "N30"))
  (pad 21 thru_hole circle (at 0 -23.876) (size 1.524 1.524) (drill 1.016) (layers *.Cu *.Mask F.SilkS) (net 31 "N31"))
  (pad 22 thru_hole circle (at -4.064 -23.876) (size 1.524 1.524) (drill 1.016) (layers *.Cu *.Mask F.SilkS) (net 36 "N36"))
  (pad 23 thru_hole circle (at -6.604 -23.876) (size 1.524 1.524) (drill 1.016) (layers *.Cu *.Mask F.SilkS) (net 37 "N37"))
  (pad 24 thru_hole circle (at -9.144 -23.876) (size 1.524 1.524) (drill 1.016) (layers *.Cu *.Mask F.SilkS) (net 38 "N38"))
  (pad 25 thru_hole circle (at -11.684 -23.876) (size 1.524 1.524) (drill 1.016) (layers *.Cu *.Mask F.SilkS) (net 39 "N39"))
  (pad 26 thru_hole circle (at -14.224 -23.876) (size 1.524 1.524) (drill 1.016) (layers *.Cu *.Mask F.SilkS) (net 48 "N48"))
  (pad 27 thru_hole circle (at -16.764 -23.876) (size 1.524 1.524) (drill 1.016) (layers *.Cu *.Mask F.SilkS) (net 49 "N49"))
  (pad 28 thru_hole circle (at -19.304 -23.876) (size 1.524 1.524) (drill 1.016) (layers *.Cu *.Mask F.SilkS))
  (pad 29 thru_hole circle (at -21.844 -23.876) (size 1.524 1.524) (drill 1.016) (layers *.Cu *.Mask F.SilkS))
  (pad 1 thru_hole circle (at -15.24 24.384) (size 1.524 1.524) (drill 1.016) (layers *.Cu *.Mask F.SilkS)))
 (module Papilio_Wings (layer F.Cu) (at 229.87 41.402 180)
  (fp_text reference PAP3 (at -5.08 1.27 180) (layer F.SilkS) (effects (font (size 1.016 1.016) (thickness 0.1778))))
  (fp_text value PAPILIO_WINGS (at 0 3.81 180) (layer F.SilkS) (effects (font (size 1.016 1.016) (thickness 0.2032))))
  (pad 1 thru_hole rect (at -21.59 -1.27 180) (size 1.524 1.524) (drill 1.016) (layers *.Cu *.Mask F.SilkS))
  (pad 7 thru_hole circle (at -6.35 -1.27 180) (size 1.524 1.524) (drill 1.016) (layers *.Cu *.Mask F.SilkS))
  (pad 2 thru_hole circle (at -19.05 -1.27 180) (size 1.524 1.524) (drill 1.016) (layers *.Cu *.Mask F.SilkS))
  (pad 8 thru_hole circle (at -3.81 -1.27 180) (size 1.524 1.524) (drill 1.016) (layers *.Cu *.Mask F.SilkS))
  (pad 3 thru_hole circle (at -16.51 -1.27 180) (size 1.524 1.524) (drill 1.016) (layers *.Cu *.Mask F.SilkS))
  (pad 9 thru_hole circle (at -1.27 -1.27 180) (size 1.524 1.524) (drill 1.016) (layers *.Cu *.Mask F.SilkS))
  (pad 4 thru_hole circle (at -13.97 -1.27 180) (size 1.524 1.524) (drill 1.016) (layers *.Cu *.Mask F.SilkS))
  (pad 10 thru_hole circle (at 1.27 -1.27 180) (size 1.524 1.524) (drill 1.016) (layers *.Cu *.Mask F.SilkS))
  (pad 5 thru_hole circle (at -11.43 -1.27 180) (size 1.524 1.524) (drill 1.016) (layers *.Cu *.Mask F.SilkS))
  (pad 11 thru_hole circle (at 3.81 -1.27 180) (size 1.524 1.524) (drill 1.016) (layers *.Cu *.Mask F.SilkS))
  (pad 6 thru_hole circle (at -8.89 -1.27 180) (size 1.524 1.524) (drill 1.016) (layers *.Cu *.Mask F.SilkS))
  (pad 12 thru_hole circle (at 6.35 -1.27 180) (size 1.524 1.524) (drill 1.016) (layers *.Cu *.Mask F.SilkS))
  (pad 13 thru_hole circle (at 8.89 -1.27 180) (size 1.524 1.524) (drill 1.016) (layers *.Cu *.Mask F.SilkS))
  (pad 14 thru_hole circle (at 11.43 -1.27 180) (size 1.524 1.524) (drill 1.016) (layers *.Cu *.Mask F.SilkS))
  (pad 15 thru_hole circle (at 13.97 -1.27 180) (size 1.524 1.524) (drill 1.016) (layers *.Cu *.Mask F.SilkS))
  (pad 16 thru_hole circle (at 16.51 -1.27 180) (size 1.524 1.524) (drill 1.016) (layers *.Cu *.Mask F.SilkS))
  (pad 17 thru_hole circle (at 6.35 1.27 180) (size 1.524 1.524) (drill 1.016) (layers *.Cu *.Mask F.SilkS))
  (pad 18 thru_hole circle (at 3.81 1.27 180) (size 1.524 1.524) (drill 1.016) (layers *.Cu *.Mask F.SilkS))
  (pad 19 thru_hole circle (at 1.27 1.27 180) (size 1.524 1.524) (drill 1.016) (layers *.Cu *.Mask F.SilkS))
  (pad 20 thru_hole circle (at -1.27 1.27 180) (size 1.524 1.524) (drill 1.016) (layers *.Cu *.Mask F.SilkS))
  (pad 21 thru_hole circle (at -13.97 1.27 180) (size 1.524 1.524) (drill 1.016) (layers *.Cu *.Mask F.SilkS))
  (pad 22 thru_hole circle (at -16.51 1.27 180) (size 1.524 1.524) (drill 1.016) (layers *.Cu *.Mask F.SilkS))
  (pad 23 thru_hole circle (at -19.05 1.27 180) (size 1.524 1.524) (drill 1.016) (layers *.Cu *.Mask F.SilkS))
  (pad 24 thru_hole circle (at -21.59 1.27 180) (size 1.524 1.524) (drill 1.016) (layers *.Cu *.Mask F.SilkS)))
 (gr_line (start 210.82 38.1) (end 210.82 102.87) (angle 90) (layer Edge.Cuts) (width 0.1))
 (gr_line (start 297.815 38.1) (end 297.815 102.87) (angle 90) (layer Edge.Cuts) (width 0.1))
 (gr_line (start 210.82 38.1) (end 297.815 38.1) (angle 90) (layer Edge.Cuts) (width 0.1))
 (gr_line (start 210.82 102.87) (end 211.455 102.87) (angle 90) (layer Edge.Cuts) (width 0.1))
 (gr_line (start 211.455 102.87) (end 297.815 102.87) (angle 90) (layer Edge.Cuts) (width 0.1))
 (segment (start 262.89 55.372) (end 262.89 49.53) (width 0.254) (layer F.Cu) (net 38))
 (segment (start 262.89 49.53) (end 262.128 48.768) (width 0.254) (layer F.Cu) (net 38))
 (segment (start 261.62 55.372) (end 261.62 50.8) (width 0.254) (layer F.Cu) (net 39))
 (segment (start 261.62 50.8) (end 259.588 48.768) (width 0.254) (layer F.Cu) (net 39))
 (segment (start 264.16 55.372) (end 264.16 49.276) (width 0.254) (layer F.Cu) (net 37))
 (segment (start 264.16 49.276) (end 264.668 48.768) (width 0.254) (layer F.Cu) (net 37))
 (segment (start 265.43 55.372) (end 265.43 50.546) (width 0.254) (layer F.Cu) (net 36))
 (segment (start 265.43 50.546) (end 267.208 48.768) (width 0.254) (layer F.Cu) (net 36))
 (segment (start 276.86 55.245) (end 276.86 49.276) (width 0.254) (layer F.Cu) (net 29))
 (segment (start 276.86 49.276) (end 276.352 48.768) (width 0.254) (layer F.Cu) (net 29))
 (segment (start 288.925 55.245) (end 288.925 51.181) (width 0.254) (layer F.Cu) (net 21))
 (segment (start 288.925 51.181) (end 286.512 48.768) (width 0.254) (layer F.Cu) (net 21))
 (segment (start 287.655 55.245) (end 287.655 52.451) (width 0.254) (layer F.Cu) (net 22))
 (segment (start 287.655 52.451) (end 283.972 48.768) (width 0.254) (layer F.Cu) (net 22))
 (segment (start 286.385 55.245) (end 286.385 53.721) (width 0.254) (layer F.Cu) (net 23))
 (segment (start 286.385 53.721) (end 281.432 48.768) (width 0.254) (layer F.Cu) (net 23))
 (segment (start 278.13 55.245) (end 278.13 49.53) (width 0.254) (layer F.Cu) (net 28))
 (segment (start 278.13 49.53) (end 278.892 48.768) (width 0.254) (layer F.Cu) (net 28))
 (segment (start 275.59 55.245) (end 275.59 50.546) (width 0.254) (layer F.Cu) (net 30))
 (segment (start 275.59 50.546) (end 273.812 48.768) (width 0.254) (layer F.Cu) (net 30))
 (segment (start 274.32 55.245) (end 274.32 51.816) (width 0.254) (layer F.Cu) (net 31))
 (segment (start 274.32 51.816) (end 271.272 48.768) (width 0.254) (layer F.Cu) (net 31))
 (segment (start 290.195 55.245) (end 290.195 49.911) (width 0.254) (layer F.Cu) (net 20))
 (segment (start 290.195 49.911) (end 289.052 48.768) (width 0.254) (layer F.Cu) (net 20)))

